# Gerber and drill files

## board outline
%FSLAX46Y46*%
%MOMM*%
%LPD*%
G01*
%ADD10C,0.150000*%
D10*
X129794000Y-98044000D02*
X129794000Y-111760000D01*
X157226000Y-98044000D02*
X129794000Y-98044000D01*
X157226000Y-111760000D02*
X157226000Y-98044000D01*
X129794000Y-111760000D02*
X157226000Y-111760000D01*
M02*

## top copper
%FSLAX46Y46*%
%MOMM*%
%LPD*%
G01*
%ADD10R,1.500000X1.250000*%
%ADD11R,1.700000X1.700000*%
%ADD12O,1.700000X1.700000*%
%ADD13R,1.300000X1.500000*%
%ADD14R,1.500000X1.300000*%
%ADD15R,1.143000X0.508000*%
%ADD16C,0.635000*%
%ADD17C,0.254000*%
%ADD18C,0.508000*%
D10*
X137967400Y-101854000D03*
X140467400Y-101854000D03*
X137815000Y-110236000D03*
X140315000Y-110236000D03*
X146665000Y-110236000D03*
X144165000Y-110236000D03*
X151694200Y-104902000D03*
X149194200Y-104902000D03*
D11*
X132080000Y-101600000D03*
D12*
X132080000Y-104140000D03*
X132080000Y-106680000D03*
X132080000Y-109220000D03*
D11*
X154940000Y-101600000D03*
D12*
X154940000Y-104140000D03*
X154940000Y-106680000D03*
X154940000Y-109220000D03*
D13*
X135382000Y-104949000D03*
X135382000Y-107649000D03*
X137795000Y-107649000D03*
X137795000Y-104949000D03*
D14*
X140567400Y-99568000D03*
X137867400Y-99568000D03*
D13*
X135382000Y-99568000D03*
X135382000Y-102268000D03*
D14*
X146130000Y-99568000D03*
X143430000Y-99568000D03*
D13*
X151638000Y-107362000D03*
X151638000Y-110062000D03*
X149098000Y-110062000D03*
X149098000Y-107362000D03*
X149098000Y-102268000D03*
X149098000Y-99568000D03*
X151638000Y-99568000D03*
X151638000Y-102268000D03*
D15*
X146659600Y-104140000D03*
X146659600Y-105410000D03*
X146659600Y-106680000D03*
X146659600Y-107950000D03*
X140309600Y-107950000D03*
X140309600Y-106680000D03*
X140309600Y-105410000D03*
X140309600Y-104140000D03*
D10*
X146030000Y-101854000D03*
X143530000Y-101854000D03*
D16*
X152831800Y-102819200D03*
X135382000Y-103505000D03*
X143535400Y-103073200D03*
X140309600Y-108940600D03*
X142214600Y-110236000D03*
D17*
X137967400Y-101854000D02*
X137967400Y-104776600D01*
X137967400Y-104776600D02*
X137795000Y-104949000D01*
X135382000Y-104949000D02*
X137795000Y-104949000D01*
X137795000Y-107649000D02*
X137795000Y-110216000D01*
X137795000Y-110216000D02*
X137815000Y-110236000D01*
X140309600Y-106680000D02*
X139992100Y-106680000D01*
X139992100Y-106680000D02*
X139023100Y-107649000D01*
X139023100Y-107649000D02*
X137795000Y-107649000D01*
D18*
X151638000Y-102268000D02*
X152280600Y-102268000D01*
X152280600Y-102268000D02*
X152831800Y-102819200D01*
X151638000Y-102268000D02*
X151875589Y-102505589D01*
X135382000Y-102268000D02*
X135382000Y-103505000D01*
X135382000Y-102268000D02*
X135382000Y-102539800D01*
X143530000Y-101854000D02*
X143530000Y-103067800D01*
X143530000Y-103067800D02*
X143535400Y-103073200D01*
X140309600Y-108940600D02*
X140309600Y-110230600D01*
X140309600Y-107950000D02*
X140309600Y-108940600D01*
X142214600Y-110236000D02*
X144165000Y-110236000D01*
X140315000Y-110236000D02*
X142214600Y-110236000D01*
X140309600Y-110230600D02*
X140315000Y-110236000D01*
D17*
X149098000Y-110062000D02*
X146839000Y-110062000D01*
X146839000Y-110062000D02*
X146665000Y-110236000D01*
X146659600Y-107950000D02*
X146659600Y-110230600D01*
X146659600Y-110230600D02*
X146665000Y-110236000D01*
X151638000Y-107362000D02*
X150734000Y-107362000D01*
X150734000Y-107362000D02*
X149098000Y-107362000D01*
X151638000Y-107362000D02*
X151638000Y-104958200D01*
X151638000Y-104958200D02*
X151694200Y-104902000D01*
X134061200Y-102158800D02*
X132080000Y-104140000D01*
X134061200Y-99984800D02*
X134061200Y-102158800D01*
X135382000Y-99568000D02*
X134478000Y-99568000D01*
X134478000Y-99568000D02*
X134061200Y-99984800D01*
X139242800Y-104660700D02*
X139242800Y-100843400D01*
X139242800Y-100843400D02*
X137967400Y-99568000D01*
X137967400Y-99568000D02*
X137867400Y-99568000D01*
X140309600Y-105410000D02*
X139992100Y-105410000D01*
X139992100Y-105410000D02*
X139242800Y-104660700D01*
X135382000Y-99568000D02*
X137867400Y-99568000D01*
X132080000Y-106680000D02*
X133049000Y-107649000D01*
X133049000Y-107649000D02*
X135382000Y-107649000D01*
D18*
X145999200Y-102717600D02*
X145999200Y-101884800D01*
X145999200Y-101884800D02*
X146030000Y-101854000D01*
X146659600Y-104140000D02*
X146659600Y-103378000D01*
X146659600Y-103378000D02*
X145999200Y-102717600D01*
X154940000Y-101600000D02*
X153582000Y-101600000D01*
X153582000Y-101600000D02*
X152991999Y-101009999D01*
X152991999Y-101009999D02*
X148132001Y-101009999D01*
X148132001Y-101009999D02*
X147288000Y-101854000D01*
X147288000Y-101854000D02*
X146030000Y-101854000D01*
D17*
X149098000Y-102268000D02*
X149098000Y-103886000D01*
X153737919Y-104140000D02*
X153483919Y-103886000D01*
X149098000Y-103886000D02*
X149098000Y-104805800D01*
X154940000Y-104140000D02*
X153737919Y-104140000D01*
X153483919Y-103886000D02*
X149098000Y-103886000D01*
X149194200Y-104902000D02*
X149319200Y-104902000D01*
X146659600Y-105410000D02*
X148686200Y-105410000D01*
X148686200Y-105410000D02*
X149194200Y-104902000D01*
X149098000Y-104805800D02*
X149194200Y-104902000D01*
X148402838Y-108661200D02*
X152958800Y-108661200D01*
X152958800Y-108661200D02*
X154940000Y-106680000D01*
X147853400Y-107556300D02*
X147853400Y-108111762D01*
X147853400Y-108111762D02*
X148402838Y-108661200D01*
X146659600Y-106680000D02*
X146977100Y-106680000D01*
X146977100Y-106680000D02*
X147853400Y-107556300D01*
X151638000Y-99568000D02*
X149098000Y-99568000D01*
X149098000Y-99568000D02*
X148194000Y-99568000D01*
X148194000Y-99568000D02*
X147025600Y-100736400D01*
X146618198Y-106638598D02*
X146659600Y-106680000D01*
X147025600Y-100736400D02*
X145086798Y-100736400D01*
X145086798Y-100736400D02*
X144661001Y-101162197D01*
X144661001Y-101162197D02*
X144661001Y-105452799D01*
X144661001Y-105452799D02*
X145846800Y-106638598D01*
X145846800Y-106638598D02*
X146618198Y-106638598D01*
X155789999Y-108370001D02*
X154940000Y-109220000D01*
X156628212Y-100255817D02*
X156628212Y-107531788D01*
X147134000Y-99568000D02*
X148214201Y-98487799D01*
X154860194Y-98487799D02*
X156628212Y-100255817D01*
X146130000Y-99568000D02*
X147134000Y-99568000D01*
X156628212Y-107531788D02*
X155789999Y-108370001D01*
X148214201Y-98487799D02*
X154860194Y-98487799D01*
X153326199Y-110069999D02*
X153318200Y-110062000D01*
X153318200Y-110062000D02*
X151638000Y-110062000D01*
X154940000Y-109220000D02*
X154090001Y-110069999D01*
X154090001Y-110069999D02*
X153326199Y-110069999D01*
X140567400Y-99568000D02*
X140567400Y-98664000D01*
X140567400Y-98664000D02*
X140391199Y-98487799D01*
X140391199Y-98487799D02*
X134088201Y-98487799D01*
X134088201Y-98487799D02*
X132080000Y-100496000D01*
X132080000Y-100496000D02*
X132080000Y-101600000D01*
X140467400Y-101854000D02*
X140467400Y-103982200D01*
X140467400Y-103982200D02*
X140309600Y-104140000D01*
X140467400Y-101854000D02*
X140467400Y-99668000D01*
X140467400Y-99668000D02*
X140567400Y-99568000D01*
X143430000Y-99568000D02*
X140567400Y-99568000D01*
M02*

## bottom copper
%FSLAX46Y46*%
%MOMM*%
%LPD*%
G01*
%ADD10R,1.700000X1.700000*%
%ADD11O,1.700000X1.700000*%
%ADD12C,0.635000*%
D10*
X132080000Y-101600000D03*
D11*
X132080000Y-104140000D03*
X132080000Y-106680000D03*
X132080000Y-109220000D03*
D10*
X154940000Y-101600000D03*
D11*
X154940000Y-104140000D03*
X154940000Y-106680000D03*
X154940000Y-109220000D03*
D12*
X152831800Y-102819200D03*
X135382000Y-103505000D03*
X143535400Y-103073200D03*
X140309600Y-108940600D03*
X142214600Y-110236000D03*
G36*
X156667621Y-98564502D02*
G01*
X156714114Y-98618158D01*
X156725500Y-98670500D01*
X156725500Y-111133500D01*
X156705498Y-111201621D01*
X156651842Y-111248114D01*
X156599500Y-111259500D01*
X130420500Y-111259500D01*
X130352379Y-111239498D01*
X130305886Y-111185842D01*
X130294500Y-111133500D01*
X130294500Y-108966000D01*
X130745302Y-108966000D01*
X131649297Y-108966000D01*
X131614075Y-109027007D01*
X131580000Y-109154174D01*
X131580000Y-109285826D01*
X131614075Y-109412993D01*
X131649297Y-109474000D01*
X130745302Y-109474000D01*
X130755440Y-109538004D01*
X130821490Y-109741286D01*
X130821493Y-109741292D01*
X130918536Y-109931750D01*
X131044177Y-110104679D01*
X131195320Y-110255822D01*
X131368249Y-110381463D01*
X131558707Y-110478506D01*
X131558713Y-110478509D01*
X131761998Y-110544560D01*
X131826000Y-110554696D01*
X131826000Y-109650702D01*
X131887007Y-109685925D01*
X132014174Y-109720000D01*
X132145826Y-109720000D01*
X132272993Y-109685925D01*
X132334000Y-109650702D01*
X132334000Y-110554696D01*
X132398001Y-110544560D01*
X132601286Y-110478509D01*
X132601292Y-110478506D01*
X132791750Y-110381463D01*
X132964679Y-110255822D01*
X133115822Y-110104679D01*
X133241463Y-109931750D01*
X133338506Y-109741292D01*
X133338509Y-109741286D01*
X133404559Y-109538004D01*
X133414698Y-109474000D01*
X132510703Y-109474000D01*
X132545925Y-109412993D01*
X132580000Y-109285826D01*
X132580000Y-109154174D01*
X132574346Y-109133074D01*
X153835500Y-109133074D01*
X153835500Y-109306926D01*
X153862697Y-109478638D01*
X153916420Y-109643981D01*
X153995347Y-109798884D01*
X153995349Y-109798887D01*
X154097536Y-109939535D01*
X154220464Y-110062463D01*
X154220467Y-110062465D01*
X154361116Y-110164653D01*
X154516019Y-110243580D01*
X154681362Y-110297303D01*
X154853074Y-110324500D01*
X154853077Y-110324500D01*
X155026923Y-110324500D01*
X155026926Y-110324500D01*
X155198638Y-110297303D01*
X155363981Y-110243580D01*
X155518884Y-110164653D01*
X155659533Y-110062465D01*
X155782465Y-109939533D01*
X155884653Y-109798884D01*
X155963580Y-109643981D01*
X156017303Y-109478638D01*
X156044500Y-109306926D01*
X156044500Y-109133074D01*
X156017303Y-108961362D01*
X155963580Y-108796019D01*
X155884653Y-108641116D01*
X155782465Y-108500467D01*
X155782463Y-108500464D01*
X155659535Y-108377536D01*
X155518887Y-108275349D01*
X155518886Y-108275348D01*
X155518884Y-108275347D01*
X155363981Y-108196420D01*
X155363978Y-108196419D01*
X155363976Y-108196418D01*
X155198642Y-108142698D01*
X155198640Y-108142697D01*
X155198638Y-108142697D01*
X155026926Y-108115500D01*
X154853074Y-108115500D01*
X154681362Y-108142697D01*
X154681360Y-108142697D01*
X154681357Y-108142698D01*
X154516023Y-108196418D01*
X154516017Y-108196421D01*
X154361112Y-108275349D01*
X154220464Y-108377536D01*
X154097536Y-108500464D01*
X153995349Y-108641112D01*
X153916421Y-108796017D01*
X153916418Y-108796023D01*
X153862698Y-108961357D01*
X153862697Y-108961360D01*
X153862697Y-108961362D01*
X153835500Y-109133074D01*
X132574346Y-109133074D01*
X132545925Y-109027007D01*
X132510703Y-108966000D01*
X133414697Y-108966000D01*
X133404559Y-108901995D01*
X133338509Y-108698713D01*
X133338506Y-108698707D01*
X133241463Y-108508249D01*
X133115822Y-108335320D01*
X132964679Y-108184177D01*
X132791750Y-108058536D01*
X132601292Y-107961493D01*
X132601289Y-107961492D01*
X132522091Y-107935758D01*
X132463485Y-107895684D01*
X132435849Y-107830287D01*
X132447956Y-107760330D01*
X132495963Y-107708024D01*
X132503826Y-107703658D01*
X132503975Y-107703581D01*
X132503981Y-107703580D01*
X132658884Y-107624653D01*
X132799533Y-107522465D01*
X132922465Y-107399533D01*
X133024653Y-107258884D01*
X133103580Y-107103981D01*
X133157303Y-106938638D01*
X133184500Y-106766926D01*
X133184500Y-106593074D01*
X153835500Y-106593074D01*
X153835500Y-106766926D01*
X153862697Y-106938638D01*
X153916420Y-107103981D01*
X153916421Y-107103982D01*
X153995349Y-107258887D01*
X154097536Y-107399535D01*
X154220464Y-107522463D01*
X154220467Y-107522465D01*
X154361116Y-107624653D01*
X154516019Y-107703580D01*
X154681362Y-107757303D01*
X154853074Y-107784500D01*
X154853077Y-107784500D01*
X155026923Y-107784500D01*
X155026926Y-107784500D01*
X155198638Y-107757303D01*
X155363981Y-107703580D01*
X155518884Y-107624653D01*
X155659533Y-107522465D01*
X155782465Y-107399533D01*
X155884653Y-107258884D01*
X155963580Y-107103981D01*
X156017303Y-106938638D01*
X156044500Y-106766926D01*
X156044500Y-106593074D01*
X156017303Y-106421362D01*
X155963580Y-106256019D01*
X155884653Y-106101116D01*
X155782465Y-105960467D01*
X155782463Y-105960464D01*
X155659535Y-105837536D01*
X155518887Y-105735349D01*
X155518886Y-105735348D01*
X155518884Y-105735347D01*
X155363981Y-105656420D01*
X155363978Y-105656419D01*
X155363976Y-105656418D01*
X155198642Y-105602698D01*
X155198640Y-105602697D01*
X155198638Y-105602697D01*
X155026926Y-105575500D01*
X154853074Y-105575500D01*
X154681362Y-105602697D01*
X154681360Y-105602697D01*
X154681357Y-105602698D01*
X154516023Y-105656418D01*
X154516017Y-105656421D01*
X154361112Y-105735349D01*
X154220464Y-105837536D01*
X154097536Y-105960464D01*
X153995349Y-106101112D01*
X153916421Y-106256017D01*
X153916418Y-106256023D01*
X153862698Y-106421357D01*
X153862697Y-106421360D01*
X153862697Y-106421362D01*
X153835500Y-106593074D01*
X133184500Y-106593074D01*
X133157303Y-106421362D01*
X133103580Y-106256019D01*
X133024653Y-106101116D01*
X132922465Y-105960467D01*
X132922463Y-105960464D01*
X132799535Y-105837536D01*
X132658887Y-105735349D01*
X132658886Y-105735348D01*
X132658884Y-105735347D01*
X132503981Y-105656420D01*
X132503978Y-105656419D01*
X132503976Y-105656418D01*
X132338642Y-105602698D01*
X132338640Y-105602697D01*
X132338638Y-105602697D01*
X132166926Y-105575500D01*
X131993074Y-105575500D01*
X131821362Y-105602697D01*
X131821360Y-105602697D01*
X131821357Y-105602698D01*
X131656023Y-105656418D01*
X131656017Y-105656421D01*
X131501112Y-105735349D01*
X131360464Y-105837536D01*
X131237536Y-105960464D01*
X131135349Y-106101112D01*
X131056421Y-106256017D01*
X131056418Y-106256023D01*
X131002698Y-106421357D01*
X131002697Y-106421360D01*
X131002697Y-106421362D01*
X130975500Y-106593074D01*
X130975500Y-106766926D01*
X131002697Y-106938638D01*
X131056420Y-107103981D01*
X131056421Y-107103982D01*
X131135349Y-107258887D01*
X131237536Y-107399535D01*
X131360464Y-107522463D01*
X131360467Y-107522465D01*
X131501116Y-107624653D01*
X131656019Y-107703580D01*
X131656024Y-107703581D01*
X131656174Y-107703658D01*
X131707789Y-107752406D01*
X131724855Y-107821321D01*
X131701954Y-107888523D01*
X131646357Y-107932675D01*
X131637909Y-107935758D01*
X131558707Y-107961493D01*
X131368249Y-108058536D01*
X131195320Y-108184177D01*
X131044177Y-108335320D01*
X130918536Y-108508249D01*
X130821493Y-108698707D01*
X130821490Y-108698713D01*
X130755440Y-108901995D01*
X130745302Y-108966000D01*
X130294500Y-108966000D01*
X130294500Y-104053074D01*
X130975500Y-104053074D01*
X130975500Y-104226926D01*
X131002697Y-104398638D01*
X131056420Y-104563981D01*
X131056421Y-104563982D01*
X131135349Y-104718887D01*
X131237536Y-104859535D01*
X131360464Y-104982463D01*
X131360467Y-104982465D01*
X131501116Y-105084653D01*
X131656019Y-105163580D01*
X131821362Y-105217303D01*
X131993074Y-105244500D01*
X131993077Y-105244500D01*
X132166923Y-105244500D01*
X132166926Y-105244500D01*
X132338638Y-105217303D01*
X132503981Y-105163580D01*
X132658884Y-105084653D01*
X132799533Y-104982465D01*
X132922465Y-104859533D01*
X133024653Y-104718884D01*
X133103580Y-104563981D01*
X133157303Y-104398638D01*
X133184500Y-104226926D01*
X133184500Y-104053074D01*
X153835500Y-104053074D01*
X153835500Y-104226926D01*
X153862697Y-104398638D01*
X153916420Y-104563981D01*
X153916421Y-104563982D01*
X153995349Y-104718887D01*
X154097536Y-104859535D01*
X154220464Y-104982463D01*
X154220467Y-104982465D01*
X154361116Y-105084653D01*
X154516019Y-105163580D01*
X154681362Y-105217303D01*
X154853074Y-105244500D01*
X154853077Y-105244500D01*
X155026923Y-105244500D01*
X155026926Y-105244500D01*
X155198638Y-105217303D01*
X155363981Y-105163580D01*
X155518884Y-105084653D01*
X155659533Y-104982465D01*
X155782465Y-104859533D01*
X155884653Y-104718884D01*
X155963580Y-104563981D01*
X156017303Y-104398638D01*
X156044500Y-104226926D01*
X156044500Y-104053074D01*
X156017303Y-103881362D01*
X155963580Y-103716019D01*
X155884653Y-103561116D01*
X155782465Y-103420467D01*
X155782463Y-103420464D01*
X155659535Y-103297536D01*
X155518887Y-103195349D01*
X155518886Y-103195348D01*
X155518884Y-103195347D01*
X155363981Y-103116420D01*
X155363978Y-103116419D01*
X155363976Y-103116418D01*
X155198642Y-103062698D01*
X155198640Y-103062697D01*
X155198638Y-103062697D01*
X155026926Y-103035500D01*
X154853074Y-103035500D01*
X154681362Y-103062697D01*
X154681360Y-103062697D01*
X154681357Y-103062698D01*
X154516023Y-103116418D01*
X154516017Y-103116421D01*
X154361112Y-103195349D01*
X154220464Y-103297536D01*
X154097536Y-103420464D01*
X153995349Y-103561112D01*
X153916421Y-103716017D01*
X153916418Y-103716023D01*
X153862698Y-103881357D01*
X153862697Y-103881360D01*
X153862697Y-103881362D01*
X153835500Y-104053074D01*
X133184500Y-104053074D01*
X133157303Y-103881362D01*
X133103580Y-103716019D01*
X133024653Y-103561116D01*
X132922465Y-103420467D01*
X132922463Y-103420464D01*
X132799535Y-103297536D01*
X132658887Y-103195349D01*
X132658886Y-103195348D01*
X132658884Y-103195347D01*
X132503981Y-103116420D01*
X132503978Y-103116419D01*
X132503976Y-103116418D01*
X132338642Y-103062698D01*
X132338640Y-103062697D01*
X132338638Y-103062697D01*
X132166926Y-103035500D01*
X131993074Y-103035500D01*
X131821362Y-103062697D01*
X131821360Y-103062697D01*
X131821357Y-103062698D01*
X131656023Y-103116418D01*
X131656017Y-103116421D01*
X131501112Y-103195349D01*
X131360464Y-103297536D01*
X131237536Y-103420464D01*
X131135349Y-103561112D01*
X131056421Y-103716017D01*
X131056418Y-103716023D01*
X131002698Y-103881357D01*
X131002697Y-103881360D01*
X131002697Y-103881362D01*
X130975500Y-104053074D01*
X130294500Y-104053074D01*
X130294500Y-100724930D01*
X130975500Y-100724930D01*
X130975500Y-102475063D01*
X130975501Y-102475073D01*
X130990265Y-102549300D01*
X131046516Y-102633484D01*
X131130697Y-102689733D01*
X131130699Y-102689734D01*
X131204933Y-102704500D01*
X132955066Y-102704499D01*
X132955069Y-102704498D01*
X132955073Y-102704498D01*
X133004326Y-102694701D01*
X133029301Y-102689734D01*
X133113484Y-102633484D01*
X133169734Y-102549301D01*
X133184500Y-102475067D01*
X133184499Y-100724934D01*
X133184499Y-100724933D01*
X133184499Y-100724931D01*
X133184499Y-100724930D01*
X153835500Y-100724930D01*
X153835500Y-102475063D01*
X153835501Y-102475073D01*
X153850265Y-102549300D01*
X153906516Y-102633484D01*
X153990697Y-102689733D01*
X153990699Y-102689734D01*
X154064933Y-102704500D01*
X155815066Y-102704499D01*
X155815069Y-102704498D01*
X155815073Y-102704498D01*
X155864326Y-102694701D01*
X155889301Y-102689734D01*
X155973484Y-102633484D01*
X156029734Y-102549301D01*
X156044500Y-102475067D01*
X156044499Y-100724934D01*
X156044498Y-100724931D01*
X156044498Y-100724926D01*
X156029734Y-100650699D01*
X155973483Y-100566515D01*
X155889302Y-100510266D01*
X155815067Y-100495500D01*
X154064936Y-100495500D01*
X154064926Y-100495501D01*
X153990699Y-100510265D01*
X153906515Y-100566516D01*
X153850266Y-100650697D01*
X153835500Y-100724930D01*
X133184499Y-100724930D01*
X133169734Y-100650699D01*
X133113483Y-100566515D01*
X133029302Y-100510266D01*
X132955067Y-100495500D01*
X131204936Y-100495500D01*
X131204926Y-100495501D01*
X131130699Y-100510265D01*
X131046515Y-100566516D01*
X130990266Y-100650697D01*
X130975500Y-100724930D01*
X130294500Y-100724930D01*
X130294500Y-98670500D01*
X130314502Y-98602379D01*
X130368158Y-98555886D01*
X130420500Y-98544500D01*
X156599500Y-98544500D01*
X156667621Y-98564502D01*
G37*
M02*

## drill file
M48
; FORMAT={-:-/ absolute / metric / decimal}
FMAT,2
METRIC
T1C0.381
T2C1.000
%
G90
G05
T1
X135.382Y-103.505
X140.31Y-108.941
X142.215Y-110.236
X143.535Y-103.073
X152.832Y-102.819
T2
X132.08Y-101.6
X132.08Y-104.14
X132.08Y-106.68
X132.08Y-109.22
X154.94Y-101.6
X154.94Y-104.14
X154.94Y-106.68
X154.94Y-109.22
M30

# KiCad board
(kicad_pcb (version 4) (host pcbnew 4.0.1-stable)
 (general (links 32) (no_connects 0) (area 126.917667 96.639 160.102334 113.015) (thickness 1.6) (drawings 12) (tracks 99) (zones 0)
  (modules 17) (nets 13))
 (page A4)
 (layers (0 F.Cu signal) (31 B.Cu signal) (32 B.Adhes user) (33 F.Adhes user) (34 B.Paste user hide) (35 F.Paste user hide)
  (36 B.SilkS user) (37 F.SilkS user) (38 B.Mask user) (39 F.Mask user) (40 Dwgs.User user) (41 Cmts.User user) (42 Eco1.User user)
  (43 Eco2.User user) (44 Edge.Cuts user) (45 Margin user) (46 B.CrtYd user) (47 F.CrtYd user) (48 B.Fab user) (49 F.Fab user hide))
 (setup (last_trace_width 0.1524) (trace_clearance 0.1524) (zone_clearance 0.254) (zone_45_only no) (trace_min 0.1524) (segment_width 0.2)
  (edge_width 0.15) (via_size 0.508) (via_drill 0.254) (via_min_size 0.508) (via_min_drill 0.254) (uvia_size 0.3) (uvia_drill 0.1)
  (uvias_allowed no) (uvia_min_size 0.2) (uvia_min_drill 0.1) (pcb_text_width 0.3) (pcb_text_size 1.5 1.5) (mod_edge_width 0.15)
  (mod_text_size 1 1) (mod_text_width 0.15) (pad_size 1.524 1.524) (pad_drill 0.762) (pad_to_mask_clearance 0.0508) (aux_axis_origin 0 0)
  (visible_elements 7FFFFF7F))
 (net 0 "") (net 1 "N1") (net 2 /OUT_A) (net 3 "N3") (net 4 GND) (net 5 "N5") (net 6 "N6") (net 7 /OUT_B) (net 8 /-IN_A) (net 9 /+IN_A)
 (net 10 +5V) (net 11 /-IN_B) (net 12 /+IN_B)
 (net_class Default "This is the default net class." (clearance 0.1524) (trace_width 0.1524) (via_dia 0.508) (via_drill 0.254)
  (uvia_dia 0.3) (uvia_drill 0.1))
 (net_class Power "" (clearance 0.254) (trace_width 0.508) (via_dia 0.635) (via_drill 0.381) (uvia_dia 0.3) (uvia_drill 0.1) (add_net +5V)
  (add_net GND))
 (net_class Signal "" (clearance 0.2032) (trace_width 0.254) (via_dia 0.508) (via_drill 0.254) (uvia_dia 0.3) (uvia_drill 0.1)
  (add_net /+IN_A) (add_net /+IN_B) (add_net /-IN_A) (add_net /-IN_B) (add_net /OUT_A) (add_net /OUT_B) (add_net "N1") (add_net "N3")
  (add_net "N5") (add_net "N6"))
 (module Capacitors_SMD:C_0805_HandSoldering (layer F.Cu) (at 139.2174 101.854)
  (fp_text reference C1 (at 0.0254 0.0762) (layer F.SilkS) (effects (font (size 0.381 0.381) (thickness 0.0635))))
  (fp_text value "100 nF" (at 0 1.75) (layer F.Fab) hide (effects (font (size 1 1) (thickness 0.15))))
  (pad 1 smd rect (at -1.25 0) (size 1.5 1.25) (layers F.Cu F.Paste F.Mask) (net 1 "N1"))
  (pad 2 smd rect (at 1.25 0) (size 1.5 1.25) (layers F.Cu F.Paste F.Mask) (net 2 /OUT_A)))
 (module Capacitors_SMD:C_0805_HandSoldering (layer F.Cu) (at 139.065 110.236)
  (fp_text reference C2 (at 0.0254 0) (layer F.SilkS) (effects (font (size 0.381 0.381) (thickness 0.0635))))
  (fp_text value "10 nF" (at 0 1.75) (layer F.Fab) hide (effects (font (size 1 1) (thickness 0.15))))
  (pad 1 smd rect (at -1.25 0) (size 1.5 1.25) (layers F.Cu F.Paste F.Mask) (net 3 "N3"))
  (pad 2 smd rect (at 1.25 0) (size 1.5 1.25) (layers F.Cu F.Paste F.Mask) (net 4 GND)))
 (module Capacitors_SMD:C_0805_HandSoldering (layer F.Cu) (at 145.415 110.236 180)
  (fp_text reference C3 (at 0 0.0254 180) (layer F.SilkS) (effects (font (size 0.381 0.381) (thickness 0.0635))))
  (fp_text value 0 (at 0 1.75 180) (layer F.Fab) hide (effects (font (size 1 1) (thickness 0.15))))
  (pad 1 smd rect (at -1.25 0 180) (size 1.5 1.25) (layers F.Cu F.Paste F.Mask) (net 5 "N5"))
  (pad 2 smd rect (at 1.25 0 180) (size 1.5 1.25) (layers F.Cu F.Paste F.Mask) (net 4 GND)))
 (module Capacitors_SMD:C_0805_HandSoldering (layer F.Cu) (at 150.4442 104.902 180)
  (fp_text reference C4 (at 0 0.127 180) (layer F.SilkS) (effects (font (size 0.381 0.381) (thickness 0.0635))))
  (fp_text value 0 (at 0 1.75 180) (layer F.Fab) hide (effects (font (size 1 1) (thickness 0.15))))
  (pad 1 smd rect (at -1.25 0 180) (size 1.5 1.25) (layers F.Cu F.Paste F.Mask) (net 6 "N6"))
  (pad 2 smd rect (at 1.25 0 180) (size 1.5 1.25) (layers F.Cu F.Paste F.Mask) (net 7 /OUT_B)))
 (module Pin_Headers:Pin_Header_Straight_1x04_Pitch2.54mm (layer F.Cu) (at 132.08 101.6)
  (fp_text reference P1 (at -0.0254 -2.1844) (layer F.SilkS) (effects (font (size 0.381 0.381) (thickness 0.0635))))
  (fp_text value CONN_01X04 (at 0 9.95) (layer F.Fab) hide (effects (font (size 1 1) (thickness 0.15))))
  (pad 1 thru_hole rect (at 0 0) (size 1.7 1.7) (drill 1) (layers *.Cu *.Mask) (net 2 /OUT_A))
  (pad 2 thru_hole oval (at 0 2.54) (size 1.7 1.7) (drill 1) (layers *.Cu *.Mask) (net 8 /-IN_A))
  (pad 3 thru_hole oval (at 0 5.08) (size 1.7 1.7) (drill 1) (layers *.Cu *.Mask) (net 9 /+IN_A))
  (pad 4 thru_hole oval (at 0 7.62) (size 1.7 1.7) (drill 1) (layers *.Cu *.Mask) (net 4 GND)))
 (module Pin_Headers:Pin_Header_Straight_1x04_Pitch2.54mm (layer F.Cu) (at 154.94 101.6)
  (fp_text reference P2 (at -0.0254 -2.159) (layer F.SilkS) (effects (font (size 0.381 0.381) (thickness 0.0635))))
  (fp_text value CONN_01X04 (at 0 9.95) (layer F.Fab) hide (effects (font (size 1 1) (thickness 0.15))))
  (pad 1 thru_hole rect (at 0 0) (size 1.7 1.7) (drill 1) (layers *.Cu *.Mask) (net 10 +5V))
  (pad 2 thru_hole oval (at 0 2.54) (size 1.7 1.7) (drill 1) (layers *.Cu *.Mask) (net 7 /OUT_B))
  (pad 3 thru_hole oval (at 0 5.08) (size 1.7 1.7) (drill 1) (layers *.Cu *.Mask) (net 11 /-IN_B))
  (pad 4 thru_hole oval (at 0 7.62) (size 1.7 1.7) (drill 1) (layers *.Cu *.Mask) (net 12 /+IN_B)))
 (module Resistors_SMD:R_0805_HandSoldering (layer F.Cu) (at 135.382 106.299 270)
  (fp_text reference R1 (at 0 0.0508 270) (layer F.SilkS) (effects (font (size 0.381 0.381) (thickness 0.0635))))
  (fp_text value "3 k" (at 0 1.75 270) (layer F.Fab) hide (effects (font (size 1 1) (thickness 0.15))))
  (pad 1 smd rect (at -1.35 0 270) (size 1.5 1.3) (layers F.Cu F.Paste F.Mask) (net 1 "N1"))
  (pad 2 smd rect (at 1.35 0 270) (size 1.5 1.3) (layers F.Cu F.Paste F.Mask) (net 9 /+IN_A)))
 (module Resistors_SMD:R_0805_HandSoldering (layer F.Cu) (at 137.795 106.299 90)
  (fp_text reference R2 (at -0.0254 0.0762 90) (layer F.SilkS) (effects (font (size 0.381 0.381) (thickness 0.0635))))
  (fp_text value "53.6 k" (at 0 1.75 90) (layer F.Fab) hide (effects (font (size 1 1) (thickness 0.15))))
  (pad 1 smd rect (at -1.35 0 90) (size 1.5 1.3) (layers F.Cu F.Paste F.Mask) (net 3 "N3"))
  (pad 2 smd rect (at 1.35 0 90) (size 1.5 1.3) (layers F.Cu F.Paste F.Mask) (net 1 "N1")))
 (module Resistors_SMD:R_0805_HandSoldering (layer F.Cu) (at 139.2174 99.568 180)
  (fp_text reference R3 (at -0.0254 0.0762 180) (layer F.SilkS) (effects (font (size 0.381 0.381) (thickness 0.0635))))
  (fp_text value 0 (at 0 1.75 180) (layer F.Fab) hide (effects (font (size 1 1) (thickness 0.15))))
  (pad 1 smd rect (at -1.35 0 180) (size 1.5 1.3) (layers F.Cu F.Paste F.Mask) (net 2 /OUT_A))
  (pad 2 smd rect (at 1.35 0 180) (size 1.5 1.3) (layers F.Cu F.Paste F.Mask) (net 8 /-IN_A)))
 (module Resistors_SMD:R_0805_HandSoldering (layer F.Cu) (at 135.382 100.918 270)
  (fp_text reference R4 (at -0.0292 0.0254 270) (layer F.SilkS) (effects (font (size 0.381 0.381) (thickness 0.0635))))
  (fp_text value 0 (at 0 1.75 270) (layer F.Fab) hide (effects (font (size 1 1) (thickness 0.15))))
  (pad 1 smd rect (at -1.35 0 270) (size 1.5 1.3) (layers F.Cu F.Paste F.Mask) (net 8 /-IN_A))
  (pad 2 smd rect (at 1.35 0 270) (size 1.5 1.3) (layers F.Cu F.Paste F.Mask) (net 4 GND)))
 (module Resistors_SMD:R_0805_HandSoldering (layer F.Cu) (at 144.78 99.568 180)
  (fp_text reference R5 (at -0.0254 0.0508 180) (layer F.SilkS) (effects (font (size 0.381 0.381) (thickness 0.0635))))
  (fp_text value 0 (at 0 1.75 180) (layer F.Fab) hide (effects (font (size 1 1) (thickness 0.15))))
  (pad 1 smd rect (at -1.35 0 180) (size 1.5 1.3) (layers F.Cu F.Paste F.Mask) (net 12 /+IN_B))
  (pad 2 smd rect (at 1.35 0 180) (size 1.5 1.3) (layers F.Cu F.Paste F.Mask) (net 2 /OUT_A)))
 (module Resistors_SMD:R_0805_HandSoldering (layer F.Cu) (at 151.638 108.712 270)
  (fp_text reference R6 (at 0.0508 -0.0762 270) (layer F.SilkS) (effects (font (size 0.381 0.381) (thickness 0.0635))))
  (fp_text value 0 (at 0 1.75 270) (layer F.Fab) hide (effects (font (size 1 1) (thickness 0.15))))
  (pad 1 smd rect (at -1.35 0 270) (size 1.5 1.3) (layers F.Cu F.Paste F.Mask) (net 6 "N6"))
  (pad 2 smd rect (at 1.35 0 270) (size 1.5 1.3) (layers F.Cu F.Paste F.Mask) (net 12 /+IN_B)))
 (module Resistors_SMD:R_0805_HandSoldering (layer F.Cu) (at 149.098 108.712 90)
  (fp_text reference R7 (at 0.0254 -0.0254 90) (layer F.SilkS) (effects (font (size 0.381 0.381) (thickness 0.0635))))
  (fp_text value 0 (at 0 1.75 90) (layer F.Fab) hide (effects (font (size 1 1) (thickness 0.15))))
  (pad 1 smd rect (at -1.35 0 90) (size 1.5 1.3) (layers F.Cu F.Paste F.Mask) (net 5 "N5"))
  (pad 2 smd rect (at 1.35 0 90) (size 1.5 1.3) (layers F.Cu F.Paste F.Mask) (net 6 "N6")))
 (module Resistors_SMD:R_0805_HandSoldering (layer F.Cu) (at 149.098 100.918 90)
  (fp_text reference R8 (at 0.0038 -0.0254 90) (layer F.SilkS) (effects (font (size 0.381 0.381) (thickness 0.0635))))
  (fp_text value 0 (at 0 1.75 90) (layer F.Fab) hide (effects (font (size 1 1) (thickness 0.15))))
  (pad 1 smd rect (at -1.35 0 90) (size 1.5 1.3) (layers F.Cu F.Paste F.Mask) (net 7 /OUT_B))
  (pad 2 smd rect (at 1.35 0 90) (size 1.5 1.3) (layers F.Cu F.Paste F.Mask) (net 11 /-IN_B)))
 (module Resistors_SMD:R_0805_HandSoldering (layer F.Cu) (at 151.638 100.918 270)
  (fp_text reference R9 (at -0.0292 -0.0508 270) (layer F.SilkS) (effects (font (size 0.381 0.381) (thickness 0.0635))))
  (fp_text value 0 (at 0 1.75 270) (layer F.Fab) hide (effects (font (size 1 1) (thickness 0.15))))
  (pad 1 smd rect (at -1.35 0 270) (size 1.5 1.3) (layers F.Cu F.Paste F.Mask) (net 11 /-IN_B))
  (pad 2 smd rect (at 1.35 0 270) (size 1.5 1.3) (layers F.Cu F.Paste F.Mask) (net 4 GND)))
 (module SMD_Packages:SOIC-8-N (layer F.Cu) (at 143.4846 106.045 270)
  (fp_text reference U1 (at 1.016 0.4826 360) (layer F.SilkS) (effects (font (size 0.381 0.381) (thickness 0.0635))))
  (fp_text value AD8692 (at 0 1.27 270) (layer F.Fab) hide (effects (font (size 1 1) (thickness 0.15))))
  (pad 8 smd rect (at -1.905 -3.175 270) (size 0.508 1.143) (layers F.Cu F.Paste F.Mask) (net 10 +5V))
  (pad 7 smd rect (at -0.635 -3.175 270) (size 0.508 1.143) (layers F.Cu F.Paste F.Mask) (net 7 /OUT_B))
  (pad 6 smd rect (at 0.635 -3.175 270) (size 0.508 1.143) (layers F.Cu F.Paste F.Mask) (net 11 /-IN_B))
  (pad 5 smd rect (at 1.905 -3.175 270) (size 0.508 1.143) (layers F.Cu F.Paste F.Mask) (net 5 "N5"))
  (pad 4 smd rect (at 1.905 3.175 270) (size 0.508 1.143) (layers F.Cu F.Paste F.Mask) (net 4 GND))
  (pad 3 smd rect (at 0.635 3.175 270) (size 0.508 1.143) (layers F.Cu F.Paste F.Mask) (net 3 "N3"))
  (pad 2 smd rect (at -0.635 3.175 270) (size 0.508 1.143) (layers F.Cu F.Paste F.Mask) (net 8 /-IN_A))
  (pad 1 smd rect (at -1.905 3.175 270) (size 0.508 1.143) (layers F.Cu F.Paste F.Mask) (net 2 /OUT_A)))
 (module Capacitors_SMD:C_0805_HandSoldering (layer F.Cu) (at 144.78 101.854 180)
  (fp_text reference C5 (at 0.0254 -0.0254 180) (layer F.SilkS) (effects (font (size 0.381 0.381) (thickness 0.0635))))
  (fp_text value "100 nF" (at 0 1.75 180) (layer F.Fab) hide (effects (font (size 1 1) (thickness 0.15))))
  (pad 1 smd rect (at -1.25 0 180) (size 1.5 1.25) (layers F.Cu F.Paste F.Mask) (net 10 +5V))
  (pad 2 smd rect (at 1.25 0 180) (size 1.5 1.25) (layers F.Cu F.Paste F.Mask) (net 4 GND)))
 (gr_line (start 129.794 98.044) (end 129.794 111.76) (layer Edge.Cuts) (width 0.15))
 (gr_line (start 157.226 98.044) (end 129.794 98.044) (layer Edge.Cuts) (width 0.15))
 (gr_line (start 157.226 111.76) (end 157.226 98.044) (layer Edge.Cuts) (width 0.15))
 (gr_line (start 129.794 111.76) (end 157.226 111.76) (layer Edge.Cuts) (width 0.15))
 (segment (start 137.9674 101.854) (end 137.9674 104.7766) (width 0.254) (layer F.Cu) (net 1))
 (segment (start 137.9674 104.7766) (end 137.795 104.949) (width 0.254) (layer F.Cu) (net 1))
 (segment (start 135.382 104.949) (end 137.795 104.949) (width 0.254) (layer F.Cu) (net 1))
 (segment (start 137.795 107.649) (end 137.795 110.216) (width 0.254) (layer F.Cu) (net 3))
 (segment (start 137.795 110.216) (end 137.815 110.236) (width 0.254) (layer F.Cu) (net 3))
 (segment (start 140.3096 106.68) (end 139.9921 106.68) (width 0.254) (layer F.Cu) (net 3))
 (segment (start 139.9921 106.68) (end 139.0231 107.649) (width 0.254) (layer F.Cu) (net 3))
 (segment (start 139.0231 107.649) (end 137.795 107.649) (width 0.254) (layer F.Cu) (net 3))
 (segment (start 151.638 102.268) (end 152.2806 102.268) (width 0.508) (layer F.Cu) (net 4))
 (segment (start 152.2806 102.268) (end 152.8318 102.8192) (width 0.508) (layer F.Cu) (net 4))
 (segment (start 151.638 102.268) (end 151.875589 102.505589) (width 0.508) (layer F.Cu) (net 4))
 (via (at 152.8318 102.8192) (size 0.635) (drill 0.381) (layers F.Cu B.Cu) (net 4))
 (segment (start 135.382 102.268) (end 135.382 103.505) (width 0.508) (layer F.Cu) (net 4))
 (via (at 135.382 103.505) (size 0.635) (drill 0.381) (layers F.Cu B.Cu) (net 4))
 (segment (start 135.382 102.268) (end 135.382 102.5398) (width 0.508) (layer F.Cu) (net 4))
 (segment (start 143.53 101.854) (end 143.53 103.0678) (width 0.508) (layer F.Cu) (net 4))
 (segment (start 143.53 103.0678) (end 143.5354 103.0732) (width 0.508) (layer F.Cu) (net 4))
 (via (at 143.5354 103.0732) (size 0.635) (drill 0.381) (layers F.Cu B.Cu) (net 4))
 (segment (start 140.3096 108.9406) (end 140.3096 110.2306) (width 0.508) (layer F.Cu) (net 4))
 (segment (start 140.3096 107.95) (end 140.3096 108.9406) (width 0.508) (layer F.Cu) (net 4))
 (via (at 140.3096 108.9406) (size 0.635) (drill 0.381) (layers F.Cu B.Cu) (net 4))
 (segment (start 142.2146 110.236) (end 144.165 110.236) (width 0.508) (layer F.Cu) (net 4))
 (segment (start 140.315 110.236) (end 142.2146 110.236) (width 0.508) (layer F.Cu) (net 4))
 (via (at 142.2146 110.236) (size 0.635) (drill 0.381) (layers F.Cu B.Cu) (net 4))
 (segment (start 140.3096 110.2306) (end 140.315 110.236) (width 0.508) (layer F.Cu) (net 4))
 (segment (start 149.098 110.062) (end 146.839 110.062) (width 0.254) (layer F.Cu) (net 5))
 (segment (start 146.839 110.062) (end 146.665 110.236) (width 0.254) (layer F.Cu) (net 5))
 (segment (start 146.6596 107.95) (end 146.6596 110.2306) (width 0.254) (layer F.Cu) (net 5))
 (segment (start 146.6596 110.2306) (end 146.665 110.236) (width 0.254) (layer F.Cu) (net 5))
 (segment (start 151.638 107.362) (end 150.734 107.362) (width 0.254) (layer F.Cu) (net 6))
 (segment (start 150.734 107.362) (end 149.098 107.362) (width 0.254) (layer F.Cu) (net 6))
 (segment (start 151.638 107.362) (end 151.638 104.9582) (width 0.254) (layer F.Cu) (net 6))
 (segment (start 151.638 104.9582) (end 151.6942 104.902) (width 0.254) (layer F.Cu) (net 6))
 (segment (start 134.0612 102.1588) (end 132.08 104.14) (width 0.254) (layer F.Cu) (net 8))
 (segment (start 134.0612 99.9848) (end 134.0612 102.1588) (width 0.254) (layer F.Cu) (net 8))
 (segment (start 135.382 99.568) (end 134.478 99.568) (width 0.254) (layer F.Cu) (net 8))
 (segment (start 134.478 99.568) (end 134.0612 99.9848) (width 0.254) (layer F.Cu) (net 8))
 (segment (start 139.2428 104.6607) (end 139.2428 100.8434) (width 0.254) (layer F.Cu) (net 8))
 (segment (start 139.2428 100.8434) (end 137.9674 99.568) (width 0.254) (layer F.Cu) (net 8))
 (segment (start 137.9674 99.568) (end 137.8674 99.568) (width 0.254) (layer F.Cu) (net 8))
 (segment (start 140.3096 105.41) (end 139.9921 105.41) (width 0.254) (layer F.Cu) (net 8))
 (segment (start 139.9921 105.41) (end 139.2428 104.6607) (width 0.254) (layer F.Cu) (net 8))
 (segment (start 135.382 99.568) (end 137.8674 99.568) (width 0.254) (layer F.Cu) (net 8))
 (segment (start 132.08 106.68) (end 133.049 107.649) (width 0.254) (layer F.Cu) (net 9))
 (segment (start 133.049 107.649) (end 135.382 107.649) (width 0.254) (layer F.Cu) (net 9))
 (segment (start 145.9992 102.7176) (end 145.9992 101.8848) (width 0.508) (layer F.Cu) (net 10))
 (segment (start 145.9992 101.8848) (end 146.03 101.854) (width 0.508) (layer F.Cu) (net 10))
 (segment (start 146.6596 104.14) (end 146.6596 103.378) (width 0.508) (layer F.Cu) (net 10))
 (segment (start 146.6596 103.378) (end 145.9992 102.7176) (width 0.508) (layer F.Cu) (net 10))
 (segment (start 154.94 101.6) (end 153.582 101.6) (width 0.508) (layer F.Cu) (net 10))
 (segment (start 153.582 101.6) (end 152.991999 101.009999) (width 0.508) (layer F.Cu) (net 10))
 (segment (start 152.991999 101.009999) (end 148.132001 101.009999) (width 0.508) (layer F.Cu) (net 10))
 (segment (start 148.132001 101.009999) (end 147.288 101.854) (width 0.508) (layer F.Cu) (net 10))
 (segment (start 147.288 101.854) (end 146.03 101.854) (width 0.508) (layer F.Cu) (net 10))
 (segment (start 149.098 102.268) (end 149.098 103.886) (width 0.254) (layer F.Cu) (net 7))
 (segment (start 153.737919 104.14) (end 153.483919 103.886) (width 0.254) (layer F.Cu) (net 7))
 (segment (start 149.098 103.886) (end 149.098 104.8058) (width 0.254) (layer F.Cu) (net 7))
 (segment (start 154.94 104.14) (end 153.737919 104.14) (width 0.254) (layer F.Cu) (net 7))
 (segment (start 153.483919 103.886) (end 149.098 103.886) (width 0.254) (layer F.Cu) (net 7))
 (segment (start 149.1942 104.902) (end 149.3192 104.902) (width 0.254) (layer F.Cu) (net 7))
 (segment (start 146.6596 105.41) (end 148.6862 105.41) (width 0.254) (layer F.Cu) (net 7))
 (segment (start 148.6862 105.41) (end 149.1942 104.902) (width 0.254) (layer F.Cu) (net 7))
 (segment (start 149.098 104.8058) (end 149.1942 104.902) (width 0.254) (layer F.Cu) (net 7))
 (segment (start 148.402838 108.6612) (end 152.9588 108.6612) (width 0.254) (layer F.Cu) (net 11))
 (segment (start 152.9588 108.6612) (end 154.94 106.68) (width 0.254) (layer F.Cu) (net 11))
 (segment (start 147.8534 107.5563) (end 147.8534 108.111762) (width 0.254) (layer F.Cu) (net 11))
 (segment (start 147.8534 108.111762) (end 148.402838 108.6612) (width 0.254) (layer F.Cu) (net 11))
 (segment (start 146.6596 106.68) (end 146.9771 106.68) (width 0.254) (layer F.Cu) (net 11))
 (segment (start 146.9771 106.68) (end 147.8534 107.5563) (width 0.254) (layer F.Cu) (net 11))
 (segment (start 151.638 99.568) (end 149.098 99.568) (width 0.254) (layer F.Cu) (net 11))
 (segment (start 149.098 99.568) (end 148.194 99.568) (width 0.254) (layer F.Cu) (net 11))
 (segment (start 148.194 99.568) (end 147.0256 100.7364) (width 0.254) (layer F.Cu) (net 11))
 (segment (start 146.618198 106.638598) (end 146.6596 106.68) (width 0.254) (layer F.Cu) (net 11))
 (segment (start 147.0256 100.7364) (end 145.086798 100.7364) (width 0.254) (layer F.Cu) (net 11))
 (segment (start 145.086798 100.7364) (end 144.661001 101.162197) (width 0.254) (layer F.Cu) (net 11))
 (segment (start 144.661001 101.162197) (end 144.661001 105.452799) (width 0.254) (layer F.Cu) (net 11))
 (segment (start 144.661001 105.452799) (end 145.8468 106.638598) (width 0.254) (layer F.Cu) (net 11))
 (segment (start 145.8468 106.638598) (end 146.618198 106.638598) (width 0.254) (layer F.Cu) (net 11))
 (segment (start 155.789999 108.370001) (end 154.94 109.22) (width 0.254) (layer F.Cu) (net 12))
 (segment (start 156.628212 100.255817) (end 156.628212 107.531788) (width 0.254) (layer F.Cu) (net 12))
 (segment (start 147.134 99.568) (end 148.214201 98.487799) (width 0.254) (layer F.Cu) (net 12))
 (segment (start 154.860194 98.487799) (end 156.628212 100.255817) (width 0.254) (layer F.Cu) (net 12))
 (segment (start 146.13 99.568) (end 147.134 99.568) (width 0.254) (layer F.Cu) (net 12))
 (segment (start 156.628212 107.531788) (end 155.789999 108.370001) (width 0.254) (layer F.Cu) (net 12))
 (segment (start 148.214201 98.487799) (end 154.860194 98.487799) (width 0.254) (layer F.Cu) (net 12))
 (segment (start 153.326199 110.069999) (end 153.3182 110.062) (width 0.254) (layer F.Cu) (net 12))
 (segment (start 153.3182 110.062) (end 151.638 110.062) (width 0.254) (layer F.Cu) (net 12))
 (segment (start 154.94 109.22) (end 154.090001 110.069999) (width 0.254) (layer F.Cu) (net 12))
 (segment (start 154.090001 110.069999) (end 153.326199 110.069999) (width 0.254) (layer F.Cu) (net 12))
 (segment (start 140.5674 99.568) (end 140.5674 98.664) (width 0.254) (layer F.Cu) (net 2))
 (segment (start 140.5674 98.664) (end 140.391199 98.487799) (width 0.254) (layer F.Cu) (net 2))
 (segment (start 140.391199 98.487799) (end 134.088201 98.487799) (width 0.254) (layer F.Cu) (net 2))
 (segment (start 134.088201 98.487799) (end 132.08 100.496) (width 0.254) (layer F.Cu) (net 2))
 (segment (start 132.08 100.496) (end 132.08 101.6) (width 0.254) (layer F.Cu) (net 2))
 (segment (start 140.4674 101.854) (end 140.4674 103.9822) (width 0.254) (layer F.Cu) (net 2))
 (segment (start 140.4674 103.9822) (end 140.3096 104.14) (width 0.254) (layer F.Cu) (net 2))
 (segment (start 140.4674 101.854) (end 140.4674 99.668) (width 0.254) (layer F.Cu) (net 2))
 (segment (start 140.4674 99.668) (end 140.5674 99.568) (width 0.254) (layer F.Cu) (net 2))
 (segment (start 143.43 99.568) (end 140.5674 99.568) (width 0.254) (layer F.Cu) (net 2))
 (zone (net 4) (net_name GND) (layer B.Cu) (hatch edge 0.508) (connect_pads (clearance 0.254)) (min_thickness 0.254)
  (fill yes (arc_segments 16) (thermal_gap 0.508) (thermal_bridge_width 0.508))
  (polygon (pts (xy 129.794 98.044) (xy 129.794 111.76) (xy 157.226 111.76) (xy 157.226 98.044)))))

